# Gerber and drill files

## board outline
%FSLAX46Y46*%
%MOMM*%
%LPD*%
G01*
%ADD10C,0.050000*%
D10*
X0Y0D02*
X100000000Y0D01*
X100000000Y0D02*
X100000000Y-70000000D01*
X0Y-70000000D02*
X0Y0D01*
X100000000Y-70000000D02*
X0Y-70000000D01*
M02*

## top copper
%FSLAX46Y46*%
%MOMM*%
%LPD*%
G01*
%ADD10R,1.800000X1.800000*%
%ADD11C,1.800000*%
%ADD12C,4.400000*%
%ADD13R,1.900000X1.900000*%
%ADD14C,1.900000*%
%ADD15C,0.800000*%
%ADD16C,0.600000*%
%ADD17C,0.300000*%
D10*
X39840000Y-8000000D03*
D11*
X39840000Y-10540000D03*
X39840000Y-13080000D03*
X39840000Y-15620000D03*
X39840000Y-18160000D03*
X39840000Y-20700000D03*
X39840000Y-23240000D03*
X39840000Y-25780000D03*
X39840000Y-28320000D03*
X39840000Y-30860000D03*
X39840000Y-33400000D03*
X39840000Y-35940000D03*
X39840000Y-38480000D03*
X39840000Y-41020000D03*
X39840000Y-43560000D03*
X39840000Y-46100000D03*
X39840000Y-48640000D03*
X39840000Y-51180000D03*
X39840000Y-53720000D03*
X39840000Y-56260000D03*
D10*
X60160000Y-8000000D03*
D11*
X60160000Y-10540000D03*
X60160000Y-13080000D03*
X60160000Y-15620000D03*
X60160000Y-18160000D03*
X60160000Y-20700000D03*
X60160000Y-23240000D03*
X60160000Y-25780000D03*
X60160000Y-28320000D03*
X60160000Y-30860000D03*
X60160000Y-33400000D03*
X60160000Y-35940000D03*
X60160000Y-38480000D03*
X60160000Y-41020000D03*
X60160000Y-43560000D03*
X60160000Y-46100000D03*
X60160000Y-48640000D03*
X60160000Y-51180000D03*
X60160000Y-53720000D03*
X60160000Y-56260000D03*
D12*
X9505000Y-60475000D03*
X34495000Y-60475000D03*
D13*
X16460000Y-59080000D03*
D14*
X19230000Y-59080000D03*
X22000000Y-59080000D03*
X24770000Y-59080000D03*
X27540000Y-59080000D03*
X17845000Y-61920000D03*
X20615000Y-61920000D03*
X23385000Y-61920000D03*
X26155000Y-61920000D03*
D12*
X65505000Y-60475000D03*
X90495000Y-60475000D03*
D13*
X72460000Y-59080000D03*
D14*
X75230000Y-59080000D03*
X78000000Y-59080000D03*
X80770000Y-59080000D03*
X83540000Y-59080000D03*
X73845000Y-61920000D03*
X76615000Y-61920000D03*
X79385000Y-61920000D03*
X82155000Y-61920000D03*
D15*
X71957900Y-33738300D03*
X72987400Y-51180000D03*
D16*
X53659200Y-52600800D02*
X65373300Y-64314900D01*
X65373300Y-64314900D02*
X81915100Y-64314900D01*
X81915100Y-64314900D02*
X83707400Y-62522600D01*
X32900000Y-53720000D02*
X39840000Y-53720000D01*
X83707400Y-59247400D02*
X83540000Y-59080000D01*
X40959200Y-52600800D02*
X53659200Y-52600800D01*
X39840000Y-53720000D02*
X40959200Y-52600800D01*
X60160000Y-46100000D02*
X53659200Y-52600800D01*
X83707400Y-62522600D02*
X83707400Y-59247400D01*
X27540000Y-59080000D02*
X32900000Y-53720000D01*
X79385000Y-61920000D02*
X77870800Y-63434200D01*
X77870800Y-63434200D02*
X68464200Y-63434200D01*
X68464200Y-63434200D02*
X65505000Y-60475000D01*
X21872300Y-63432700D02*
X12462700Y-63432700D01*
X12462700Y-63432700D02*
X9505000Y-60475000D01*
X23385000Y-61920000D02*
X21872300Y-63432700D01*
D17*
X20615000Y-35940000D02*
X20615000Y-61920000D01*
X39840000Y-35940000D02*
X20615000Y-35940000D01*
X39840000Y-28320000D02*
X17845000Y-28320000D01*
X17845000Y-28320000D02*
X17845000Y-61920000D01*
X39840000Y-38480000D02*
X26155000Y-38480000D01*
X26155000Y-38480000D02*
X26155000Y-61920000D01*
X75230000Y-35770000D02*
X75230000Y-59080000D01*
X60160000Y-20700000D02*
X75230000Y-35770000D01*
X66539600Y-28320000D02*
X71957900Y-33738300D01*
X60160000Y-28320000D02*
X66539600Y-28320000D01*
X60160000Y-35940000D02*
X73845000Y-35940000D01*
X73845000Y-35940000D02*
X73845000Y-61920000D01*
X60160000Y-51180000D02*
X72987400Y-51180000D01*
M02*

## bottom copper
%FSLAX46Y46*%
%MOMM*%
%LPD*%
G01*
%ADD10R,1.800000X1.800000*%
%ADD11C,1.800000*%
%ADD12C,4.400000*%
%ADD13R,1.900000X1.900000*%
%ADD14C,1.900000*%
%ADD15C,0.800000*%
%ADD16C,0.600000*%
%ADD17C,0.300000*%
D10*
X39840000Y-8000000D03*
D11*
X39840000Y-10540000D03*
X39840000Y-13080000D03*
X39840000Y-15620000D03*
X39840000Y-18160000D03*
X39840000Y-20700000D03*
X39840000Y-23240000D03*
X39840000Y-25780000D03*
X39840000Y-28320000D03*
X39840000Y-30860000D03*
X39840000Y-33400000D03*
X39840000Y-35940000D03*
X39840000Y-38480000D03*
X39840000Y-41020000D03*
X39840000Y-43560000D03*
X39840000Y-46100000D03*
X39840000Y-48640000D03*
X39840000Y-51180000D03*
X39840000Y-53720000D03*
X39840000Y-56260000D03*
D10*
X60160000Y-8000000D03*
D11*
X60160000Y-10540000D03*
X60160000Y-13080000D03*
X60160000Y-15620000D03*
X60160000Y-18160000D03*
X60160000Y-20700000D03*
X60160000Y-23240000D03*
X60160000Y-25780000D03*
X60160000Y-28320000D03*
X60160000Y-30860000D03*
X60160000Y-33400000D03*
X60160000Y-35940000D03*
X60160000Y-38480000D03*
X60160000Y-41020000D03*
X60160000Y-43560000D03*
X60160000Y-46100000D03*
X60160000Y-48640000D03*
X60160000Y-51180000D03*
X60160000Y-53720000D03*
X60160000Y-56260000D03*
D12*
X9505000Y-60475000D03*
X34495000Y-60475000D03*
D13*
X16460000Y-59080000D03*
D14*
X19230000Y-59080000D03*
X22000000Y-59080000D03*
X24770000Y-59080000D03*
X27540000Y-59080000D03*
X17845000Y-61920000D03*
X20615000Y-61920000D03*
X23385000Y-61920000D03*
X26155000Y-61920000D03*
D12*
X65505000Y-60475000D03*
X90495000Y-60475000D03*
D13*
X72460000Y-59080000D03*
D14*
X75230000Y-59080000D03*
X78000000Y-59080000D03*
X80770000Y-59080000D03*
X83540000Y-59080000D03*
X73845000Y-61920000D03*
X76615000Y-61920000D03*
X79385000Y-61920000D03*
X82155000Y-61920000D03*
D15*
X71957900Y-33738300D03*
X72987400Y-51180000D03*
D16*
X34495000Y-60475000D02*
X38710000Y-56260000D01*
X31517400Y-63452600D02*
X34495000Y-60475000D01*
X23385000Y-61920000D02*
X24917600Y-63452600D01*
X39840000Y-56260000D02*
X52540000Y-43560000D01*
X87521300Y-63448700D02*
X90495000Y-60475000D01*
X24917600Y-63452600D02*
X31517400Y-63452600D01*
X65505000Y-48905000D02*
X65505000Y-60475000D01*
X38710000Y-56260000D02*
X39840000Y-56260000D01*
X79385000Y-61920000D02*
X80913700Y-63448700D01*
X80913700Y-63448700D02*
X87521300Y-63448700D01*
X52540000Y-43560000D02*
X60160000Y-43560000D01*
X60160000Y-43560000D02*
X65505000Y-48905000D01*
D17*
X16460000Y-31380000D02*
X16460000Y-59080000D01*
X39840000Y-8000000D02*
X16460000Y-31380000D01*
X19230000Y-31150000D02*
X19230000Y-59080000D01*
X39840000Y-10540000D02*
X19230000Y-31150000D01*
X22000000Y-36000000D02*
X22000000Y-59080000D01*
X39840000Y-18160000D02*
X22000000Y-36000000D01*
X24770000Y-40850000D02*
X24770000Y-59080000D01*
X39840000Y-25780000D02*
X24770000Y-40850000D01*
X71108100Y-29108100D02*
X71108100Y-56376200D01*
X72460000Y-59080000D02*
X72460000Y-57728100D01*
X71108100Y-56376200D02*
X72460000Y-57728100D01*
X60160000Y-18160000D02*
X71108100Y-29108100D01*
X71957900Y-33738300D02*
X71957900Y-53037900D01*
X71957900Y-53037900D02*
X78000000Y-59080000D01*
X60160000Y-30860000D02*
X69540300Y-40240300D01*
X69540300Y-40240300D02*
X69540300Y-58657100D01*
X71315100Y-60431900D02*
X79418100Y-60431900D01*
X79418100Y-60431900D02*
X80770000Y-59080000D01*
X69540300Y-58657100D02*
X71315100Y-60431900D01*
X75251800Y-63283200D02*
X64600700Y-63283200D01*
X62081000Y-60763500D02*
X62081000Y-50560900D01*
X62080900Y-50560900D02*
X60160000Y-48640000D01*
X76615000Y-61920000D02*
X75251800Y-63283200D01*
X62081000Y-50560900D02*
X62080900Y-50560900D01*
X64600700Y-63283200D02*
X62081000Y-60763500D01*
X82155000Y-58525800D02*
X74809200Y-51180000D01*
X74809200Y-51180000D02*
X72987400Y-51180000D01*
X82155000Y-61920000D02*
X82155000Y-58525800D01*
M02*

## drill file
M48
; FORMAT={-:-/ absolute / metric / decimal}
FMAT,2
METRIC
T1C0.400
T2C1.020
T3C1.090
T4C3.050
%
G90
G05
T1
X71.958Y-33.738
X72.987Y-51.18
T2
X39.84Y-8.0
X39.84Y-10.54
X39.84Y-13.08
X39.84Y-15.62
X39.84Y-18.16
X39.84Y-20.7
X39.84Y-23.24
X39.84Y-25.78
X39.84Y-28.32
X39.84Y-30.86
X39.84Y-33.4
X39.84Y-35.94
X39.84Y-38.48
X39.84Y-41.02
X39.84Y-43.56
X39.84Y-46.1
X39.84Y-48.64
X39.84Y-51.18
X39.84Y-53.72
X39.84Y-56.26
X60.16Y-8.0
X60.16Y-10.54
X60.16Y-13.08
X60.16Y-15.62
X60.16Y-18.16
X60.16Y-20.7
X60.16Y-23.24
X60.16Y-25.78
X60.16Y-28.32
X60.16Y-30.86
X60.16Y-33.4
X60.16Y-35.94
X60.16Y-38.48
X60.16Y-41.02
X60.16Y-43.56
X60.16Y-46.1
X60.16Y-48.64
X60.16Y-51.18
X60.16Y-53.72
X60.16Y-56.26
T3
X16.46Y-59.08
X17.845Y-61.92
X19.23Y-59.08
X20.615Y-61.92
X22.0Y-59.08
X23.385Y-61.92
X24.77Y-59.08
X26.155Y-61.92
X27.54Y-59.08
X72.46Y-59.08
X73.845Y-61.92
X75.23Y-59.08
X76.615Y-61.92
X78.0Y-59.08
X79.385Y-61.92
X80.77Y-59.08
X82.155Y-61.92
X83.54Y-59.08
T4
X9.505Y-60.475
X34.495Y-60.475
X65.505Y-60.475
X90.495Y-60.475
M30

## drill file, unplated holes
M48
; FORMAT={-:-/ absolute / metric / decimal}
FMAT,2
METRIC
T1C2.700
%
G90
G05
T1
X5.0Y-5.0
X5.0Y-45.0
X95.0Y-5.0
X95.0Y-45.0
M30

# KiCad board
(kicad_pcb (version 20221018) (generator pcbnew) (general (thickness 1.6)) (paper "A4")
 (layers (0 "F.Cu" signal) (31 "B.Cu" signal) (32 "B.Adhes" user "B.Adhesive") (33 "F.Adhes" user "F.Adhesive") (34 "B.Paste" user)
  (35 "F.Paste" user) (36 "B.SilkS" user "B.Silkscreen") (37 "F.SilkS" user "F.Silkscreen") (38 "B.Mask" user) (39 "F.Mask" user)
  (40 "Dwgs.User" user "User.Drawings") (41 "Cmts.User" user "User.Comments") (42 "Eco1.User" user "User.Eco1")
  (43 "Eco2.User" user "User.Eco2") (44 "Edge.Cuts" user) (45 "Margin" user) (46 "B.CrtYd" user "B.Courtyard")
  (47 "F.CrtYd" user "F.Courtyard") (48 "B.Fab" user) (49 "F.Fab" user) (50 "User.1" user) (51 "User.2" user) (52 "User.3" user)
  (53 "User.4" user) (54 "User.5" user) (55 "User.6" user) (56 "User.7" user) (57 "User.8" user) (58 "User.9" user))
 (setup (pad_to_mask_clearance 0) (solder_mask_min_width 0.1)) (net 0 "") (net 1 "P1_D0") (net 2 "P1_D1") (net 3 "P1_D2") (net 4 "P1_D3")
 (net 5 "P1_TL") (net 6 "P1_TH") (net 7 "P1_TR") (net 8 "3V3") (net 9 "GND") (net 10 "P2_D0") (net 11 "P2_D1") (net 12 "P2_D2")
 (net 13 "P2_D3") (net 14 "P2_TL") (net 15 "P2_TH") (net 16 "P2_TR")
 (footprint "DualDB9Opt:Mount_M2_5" (layer "F.Cu") (at 95 45)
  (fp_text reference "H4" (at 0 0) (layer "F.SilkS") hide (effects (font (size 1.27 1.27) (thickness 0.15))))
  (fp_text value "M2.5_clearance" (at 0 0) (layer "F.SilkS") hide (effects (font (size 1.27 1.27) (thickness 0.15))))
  (pad "" np_thru_hole circle (at 0 0) (size 2.7 2.7) (drill 2.7) (layers "F&B.Cu" "*.Mask")))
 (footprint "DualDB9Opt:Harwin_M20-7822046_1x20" (layer "F.Cu") (at 39.84 8)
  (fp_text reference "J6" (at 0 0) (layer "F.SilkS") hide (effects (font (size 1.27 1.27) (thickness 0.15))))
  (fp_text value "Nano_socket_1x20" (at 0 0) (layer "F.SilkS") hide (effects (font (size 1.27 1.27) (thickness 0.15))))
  (pad "1" thru_hole rect (at 0 0) (size 1.8 1.8) (drill 1.02) (layers "F&B.Cu" "*.Mask") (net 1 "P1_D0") (thermal_bridge_angle 45))
  (pad "2" thru_hole circle (at 0 2.54) (size 1.8 1.8) (drill 1.02) (layers "F&B.Cu" "*.Mask") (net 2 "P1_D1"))
  (pad "3" thru_hole circle (at 0 5.08) (size 1.8 1.8) (drill 1.02) (layers "F&B.Cu" "*.Mask"))
  (pad "4" thru_hole circle (at 0 7.62) (size 1.8 1.8) (drill 1.02) (layers "F&B.Cu" "*.Mask"))
  (pad "5" thru_hole circle (at 0 10.16) (size 1.8 1.8) (drill 1.02) (layers "F&B.Cu" "*.Mask") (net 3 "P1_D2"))
  (pad "6" thru_hole circle (at 0 12.7) (size 1.8 1.8) (drill 1.02) (layers "F&B.Cu" "*.Mask"))
  (pad "7" thru_hole circle (at 0 15.24) (size 1.8 1.8) (drill 1.02) (layers "F&B.Cu" "*.Mask"))
  (pad "8" thru_hole circle (at 0 17.78) (size 1.8 1.8) (drill 1.02) (layers "F&B.Cu" "*.Mask") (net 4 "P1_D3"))
  (pad "9" thru_hole circle (at 0 20.32) (size 1.8 1.8) (drill 1.02) (layers "F&B.Cu" "*.Mask") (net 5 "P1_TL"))
  (pad "10" thru_hole circle (at 0 22.86) (size 1.8 1.8) (drill 1.02) (layers "F&B.Cu" "*.Mask"))
  (pad "11" thru_hole circle (at 0 25.4) (size 1.8 1.8) (drill 1.02) (layers "F&B.Cu" "*.Mask"))
  (pad "12" thru_hole circle (at 0 27.94) (size 1.8 1.8) (drill 1.02) (layers "F&B.Cu" "*.Mask") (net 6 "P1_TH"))
  (pad "13" thru_hole circle (at 0 30.48) (size 1.8 1.8) (drill 1.02) (layers "F&B.Cu" "*.Mask") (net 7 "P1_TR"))
  (pad "14" thru_hole circle (at 0 33.02) (size 1.8 1.8) (drill 1.02) (layers "F&B.Cu" "*.Mask"))
  (pad "15" thru_hole circle (at 0 35.56) (size 1.8 1.8) (drill 1.02) (layers "F&B.Cu" "*.Mask"))
  (pad "16" thru_hole circle (at 0 38.1) (size 1.8 1.8) (drill 1.02) (layers "F&B.Cu" "*.Mask"))
  (pad "17" thru_hole circle (at 0 40.64) (size 1.8 1.8) (drill 1.02) (layers "F&B.Cu" "*.Mask"))
  (pad "18" thru_hole circle (at 0 43.18) (size 1.8 1.8) (drill 1.02) (layers "F&B.Cu" "*.Mask"))
  (pad "19" thru_hole circle (at 0 45.72) (size 1.8 1.8) (drill 1.02) (layers "F&B.Cu" "*.Mask") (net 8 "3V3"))
  (pad "20" thru_hole circle (at 0 48.26) (size 1.8 1.8) (drill 1.02) (layers "F&B.Cu" "*.Mask") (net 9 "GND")))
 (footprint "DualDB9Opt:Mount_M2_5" (layer "F.Cu") (at 5 5)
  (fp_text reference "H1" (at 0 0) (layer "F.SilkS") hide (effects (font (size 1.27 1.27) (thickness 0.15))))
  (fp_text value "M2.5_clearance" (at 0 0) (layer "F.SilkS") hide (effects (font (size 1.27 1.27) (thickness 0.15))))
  (pad "" np_thru_hole circle (at 0 0) (size 2.7 2.7) (drill 2.7) (layers "F&B.Cu" "*.Mask")))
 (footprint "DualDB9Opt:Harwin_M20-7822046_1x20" (layer "F.Cu") (at 60.16 8)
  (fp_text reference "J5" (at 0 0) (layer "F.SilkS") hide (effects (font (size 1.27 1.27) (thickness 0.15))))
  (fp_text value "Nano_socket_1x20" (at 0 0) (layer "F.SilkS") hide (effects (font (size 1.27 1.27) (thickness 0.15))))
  (pad "1" thru_hole rect (at 0 0) (size 1.8 1.8) (drill 1.02) (layers "F&B.Cu" "*.Mask") (thermal_bridge_angle 45))
  (pad "2" thru_hole circle (at 0 2.54) (size 1.8 1.8) (drill 1.02) (layers "F&B.Cu" "*.Mask"))
  (pad "3" thru_hole circle (at 0 5.08) (size 1.8 1.8) (drill 1.02) (layers "F&B.Cu" "*.Mask"))
  (pad "4" thru_hole circle (at 0 7.62) (size 1.8 1.8) (drill 1.02) (layers "F&B.Cu" "*.Mask"))
  (pad "5" thru_hole circle (at 0 10.16) (size 1.8 1.8) (drill 1.02) (layers "F&B.Cu" "*.Mask") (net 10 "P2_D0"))
  (pad "6" thru_hole circle (at 0 12.7) (size 1.8 1.8) (drill 1.02) (layers "F&B.Cu" "*.Mask") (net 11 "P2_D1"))
  (pad "7" thru_hole circle (at 0 15.24) (size 1.8 1.8) (drill 1.02) (layers "F&B.Cu" "*.Mask"))
  (pad "8" thru_hole circle (at 0 17.78) (size 1.8 1.8) (drill 1.02) (layers "F&B.Cu" "*.Mask"))
  (pad "9" thru_hole circle (at 0 20.32) (size 1.8 1.8) (drill 1.02) (layers "F&B.Cu" "*.Mask") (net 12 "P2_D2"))
  (pad "10" thru_hole circle (at 0 22.86) (size 1.8 1.8) (drill 1.02) (layers "F&B.Cu" "*.Mask") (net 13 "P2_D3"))
  (pad "11" thru_hole circle (at 0 25.4) (size 1.8 1.8) (drill 1.02) (layers "F&B.Cu" "*.Mask"))
  (pad "12" thru_hole circle (at 0 27.94) (size 1.8 1.8) (drill 1.02) (layers "F&B.Cu" "*.Mask") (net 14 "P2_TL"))
  (pad "13" thru_hole circle (at 0 30.48) (size 1.8 1.8) (drill 1.02) (layers "F&B.Cu" "*.Mask"))
  (pad "14" thru_hole circle (at 0 33.02) (size 1.8 1.8) (drill 1.02) (layers "F&B.Cu" "*.Mask"))
  (pad "15" thru_hole circle (at 0 35.56) (size 1.8 1.8) (drill 1.02) (layers "F&B.Cu" "*.Mask") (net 9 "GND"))
  (pad "16" thru_hole circle (at 0 38.1) (size 1.8 1.8) (drill 1.02) (layers "F&B.Cu" "*.Mask") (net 8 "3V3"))
  (pad "17" thru_hole circle (at 0 40.64) (size 1.8 1.8) (drill 1.02) (layers "F&B.Cu" "*.Mask") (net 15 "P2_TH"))
  (pad "18" thru_hole circle (at 0 43.18) (size 1.8 1.8) (drill 1.02) (layers "F&B.Cu" "*.Mask") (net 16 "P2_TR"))
  (pad "19" thru_hole circle (at 0 45.72) (size 1.8 1.8) (drill 1.02) (layers "F&B.Cu" "*.Mask"))
  (pad "20" thru_hole circle (at 0 48.26) (size 1.8 1.8) (drill 1.02) (layers "F&B.Cu" "*.Mask")))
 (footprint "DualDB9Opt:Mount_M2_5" (layer "F.Cu") (at 5 45)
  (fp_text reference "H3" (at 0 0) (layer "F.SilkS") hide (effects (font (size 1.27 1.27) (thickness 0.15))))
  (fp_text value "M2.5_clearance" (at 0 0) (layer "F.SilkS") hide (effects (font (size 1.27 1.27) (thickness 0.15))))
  (pad "" np_thru_hole circle (at 0 0) (size 2.7 2.7) (drill 2.7) (layers "F&B.Cu" "*.Mask")))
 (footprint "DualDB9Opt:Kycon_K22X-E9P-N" (layer "F.Cu") (at 16.46 59.08)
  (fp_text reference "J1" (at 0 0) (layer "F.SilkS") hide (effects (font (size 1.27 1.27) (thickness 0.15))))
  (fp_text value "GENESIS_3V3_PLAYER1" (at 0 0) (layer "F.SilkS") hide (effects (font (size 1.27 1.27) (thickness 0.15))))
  (pad "0" thru_hole circle (at -6.955 1.395) (size 4.4 4.4) (drill 3.05) (layers "F&B.Cu" "*.Mask") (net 9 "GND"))
  (pad "0" thru_hole circle (at 18.035 1.395) (size 4.4 4.4) (drill 3.05) (layers "F&B.Cu" "*.Mask") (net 9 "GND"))
  (pad "1" thru_hole rect (at 0 0) (size 1.9 1.9) (drill 1.09) (layers "F&B.Cu" "*.Mask") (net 1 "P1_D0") (thermal_bridge_angle 45))
  (pad "2" thru_hole circle (at 2.77 0) (size 1.9 1.9) (drill 1.09) (layers "F&B.Cu" "*.Mask") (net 2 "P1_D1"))
  (pad "3" thru_hole circle (at 5.54 0) (size 1.9 1.9) (drill 1.09) (layers "F&B.Cu" "*.Mask") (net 3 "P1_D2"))
  (pad "4" thru_hole circle (at 8.31 0) (size 1.9 1.9) (drill 1.09) (layers "F&B.Cu" "*.Mask") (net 4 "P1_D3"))
  (pad "5" thru_hole circle (at 11.08 0) (size 1.9 1.9) (drill 1.09) (layers "F&B.Cu" "*.Mask") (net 8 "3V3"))
  (pad "6" thru_hole circle (at 1.385 2.84) (size 1.9 1.9) (drill 1.09) (layers "F&B.Cu" "*.Mask") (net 5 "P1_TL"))
  (pad "7" thru_hole circle (at 4.155 2.84) (size 1.9 1.9) (drill 1.09) (layers "F&B.Cu" "*.Mask") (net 6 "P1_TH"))
  (pad "8" thru_hole circle (at 6.925 2.84) (size 1.9 1.9) (drill 1.09) (layers "F&B.Cu" "*.Mask") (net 9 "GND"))
  (pad "9" thru_hole circle (at 9.695 2.84) (size 1.9 1.9) (drill 1.09) (layers "F&B.Cu" "*.Mask") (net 7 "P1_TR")))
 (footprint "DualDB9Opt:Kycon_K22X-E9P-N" (layer "F.Cu") (at 72.46 59.08)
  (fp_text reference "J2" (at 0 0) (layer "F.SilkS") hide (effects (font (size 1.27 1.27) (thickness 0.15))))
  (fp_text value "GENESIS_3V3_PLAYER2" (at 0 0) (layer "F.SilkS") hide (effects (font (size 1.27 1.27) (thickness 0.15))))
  (pad "0" thru_hole circle (at -6.955 1.395) (size 4.4 4.4) (drill 3.05) (layers "F&B.Cu" "*.Mask") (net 9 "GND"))
  (pad "0" thru_hole circle (at 18.035 1.395) (size 4.4 4.4) (drill 3.05) (layers "F&B.Cu" "*.Mask") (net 9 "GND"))
  (pad "1" thru_hole rect (at 0 0) (size 1.9 1.9) (drill 1.09) (layers "F&B.Cu" "*.Mask") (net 10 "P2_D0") (thermal_bridge_angle 45))
  (pad "2" thru_hole circle (at 2.77 0) (size 1.9 1.9) (drill 1.09) (layers "F&B.Cu" "*.Mask") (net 11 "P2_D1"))
  (pad "3" thru_hole circle (at 5.54 0) (size 1.9 1.9) (drill 1.09) (layers "F&B.Cu" "*.Mask") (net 12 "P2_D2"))
  (pad "4" thru_hole circle (at 8.31 0) (size 1.9 1.9) (drill 1.09) (layers "F&B.Cu" "*.Mask") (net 13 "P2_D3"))
  (pad "5" thru_hole circle (at 11.08 0) (size 1.9 1.9) (drill 1.09) (layers "F&B.Cu" "*.Mask") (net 8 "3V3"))
  (pad "6" thru_hole circle (at 1.385 2.84) (size 1.9 1.9) (drill 1.09) (layers "F&B.Cu" "*.Mask") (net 14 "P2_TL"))
  (pad "7" thru_hole circle (at 4.155 2.84) (size 1.9 1.9) (drill 1.09) (layers "F&B.Cu" "*.Mask") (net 15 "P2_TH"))
  (pad "8" thru_hole circle (at 6.925 2.84) (size 1.9 1.9) (drill 1.09) (layers "F&B.Cu" "*.Mask") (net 9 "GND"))
  (pad "9" thru_hole circle (at 9.695 2.84) (size 1.9 1.9) (drill 1.09) (layers "F&B.Cu" "*.Mask") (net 16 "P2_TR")))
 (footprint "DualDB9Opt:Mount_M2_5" (layer "F.Cu") (at 95 5)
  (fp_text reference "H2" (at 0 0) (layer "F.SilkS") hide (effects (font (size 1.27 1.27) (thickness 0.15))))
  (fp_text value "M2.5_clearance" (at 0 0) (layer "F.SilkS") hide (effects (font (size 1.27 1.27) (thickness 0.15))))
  (pad "" np_thru_hole circle (at 0 0) (size 2.7 2.7) (drill 2.7) (layers "F&B.Cu" "*.Mask")))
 (gr_line (start 0 0) (end 100 0) (stroke (width 0.05) (type default)) (layer "Edge.Cuts"))
 (gr_line (start 100 0) (end 100 70) (stroke (width 0.05) (type default)) (layer "Edge.Cuts"))
 (gr_line (start 0 70) (end 0 0) (stroke (width 0.05) (type default)) (layer "Edge.Cuts"))
 (gr_line (start 100 70) (end 0 70) (stroke (width 0.05) (type default)) (layer "Edge.Cuts"))
 (segment (start 53.6592 52.6008) (end 65.3733 64.3149) (width 0.6) (layer "F.Cu") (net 8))
 (segment (start 65.3733 64.3149) (end 81.9151 64.3149) (width 0.6) (layer "F.Cu") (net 8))
 (segment (start 81.9151 64.3149) (end 83.7074 62.5226) (width 0.6) (layer "F.Cu") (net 8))
 (segment (start 32.9 53.72) (end 39.84 53.72) (width 0.6) (layer "F.Cu") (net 8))
 (segment (start 83.7074 59.2474) (end 83.54 59.08) (width 0.6) (layer "F.Cu") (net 8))
 (segment (start 40.9592 52.6008) (end 53.6592 52.6008) (width 0.6) (layer "F.Cu") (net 8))
 (segment (start 39.84 53.72) (end 40.9592 52.6008) (width 0.6) (layer "F.Cu") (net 8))
 (segment (start 60.16 46.1) (end 53.6592 52.6008) (width 0.6) (layer "F.Cu") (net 8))
 (segment (start 83.7074 62.5226) (end 83.7074 59.2474) (width 0.6) (layer "F.Cu") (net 8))
 (segment (start 27.54 59.08) (end 32.9 53.72) (width 0.6) (layer "F.Cu") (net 8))
 (segment (start 79.385 61.92) (end 77.8708 63.4342) (width 0.6) (layer "F.Cu") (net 9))
 (segment (start 77.8708 63.4342) (end 68.4642 63.4342) (width 0.6) (layer "F.Cu") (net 9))
 (segment (start 68.4642 63.4342) (end 65.505 60.475) (width 0.6) (layer "F.Cu") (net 9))
 (segment (start 21.8723 63.4327) (end 12.4627 63.4327) (width 0.6) (layer "F.Cu") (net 9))
 (segment (start 12.4627 63.4327) (end 9.505 60.475) (width 0.6) (layer "F.Cu") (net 9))
 (segment (start 23.385 61.92) (end 21.8723 63.4327) (width 0.6) (layer "F.Cu") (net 9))
 (segment (start 34.495 60.475) (end 38.71 56.26) (width 0.6) (layer "B.Cu") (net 9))
 (segment (start 31.5174 63.4526) (end 34.495 60.475) (width 0.6) (layer "B.Cu") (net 9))
 (segment (start 23.385 61.92) (end 24.9176 63.4526) (width 0.6) (layer "B.Cu") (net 9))
 (segment (start 39.84 56.26) (end 52.54 43.56) (width 0.6) (layer "B.Cu") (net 9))
 (segment (start 87.5213 63.4487) (end 90.495 60.475) (width 0.6) (layer "B.Cu") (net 9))
 (segment (start 24.9176 63.4526) (end 31.5174 63.4526) (width 0.6) (layer "B.Cu") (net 9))
 (segment (start 65.505 48.905) (end 65.505 60.475) (width 0.6) (layer "B.Cu") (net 9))
 (segment (start 38.71 56.26) (end 39.84 56.26) (width 0.6) (layer "B.Cu") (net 9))
 (segment (start 79.385 61.92) (end 80.9137 63.4487) (width 0.6) (layer "B.Cu") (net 9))
 (segment (start 80.9137 63.4487) (end 87.5213 63.4487) (width 0.6) (layer "B.Cu") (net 9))
 (segment (start 52.54 43.56) (end 60.16 43.56) (width 0.6) (layer "B.Cu") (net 9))
 (segment (start 60.16 43.56) (end 65.505 48.905) (width 0.6) (layer "B.Cu") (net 9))
 (segment (start 16.46 31.38) (end 16.46 59.08) (width 0.3) (layer "B.Cu") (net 1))
 (segment (start 39.84 8) (end 16.46 31.38) (width 0.3) (layer "B.Cu") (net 1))
 (segment (start 19.23 31.15) (end 19.23 59.08) (width 0.3) (layer "B.Cu") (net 2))
 (segment (start 39.84 10.54) (end 19.23 31.15) (width 0.3) (layer "B.Cu") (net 2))
 (segment (start 22 36) (end 22 59.08) (width 0.3) (layer "B.Cu") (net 3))
 (segment (start 39.84 18.16) (end 22 36) (width 0.3) (layer "B.Cu") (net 3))
 (segment (start 24.77 40.85) (end 24.77 59.08) (width 0.3) (layer "B.Cu") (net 4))
 (segment (start 39.84 25.78) (end 24.77 40.85) (width 0.3) (layer "B.Cu") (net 4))
 (segment (start 20.615 35.94) (end 20.615 61.92) (width 0.3) (layer "F.Cu") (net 6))
 (segment (start 39.84 35.94) (end 20.615 35.94) (width 0.3) (layer "F.Cu") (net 6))
 (segment (start 39.84 28.32) (end 17.845 28.32) (width 0.3) (layer "F.Cu") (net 5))
 (segment (start 17.845 28.32) (end 17.845 61.92) (width 0.3) (layer "F.Cu") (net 5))
 (segment (start 39.84 38.48) (end 26.155 38.48) (width 0.3) (layer "F.Cu") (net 7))
 (segment (start 26.155 38.48) (end 26.155 61.92) (width 0.3) (layer "F.Cu") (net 7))
 (segment (start 71.1081 29.1081) (end 71.1081 56.3762) (width 0.3) (layer "B.Cu") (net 10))
 (segment (start 72.46 59.08) (end 72.46 57.7281) (width 0.3) (layer "B.Cu") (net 10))
 (segment (start 71.1081 56.3762) (end 72.46 57.7281) (width 0.3) (layer "B.Cu") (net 10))
 (segment (start 60.16 18.16) (end 71.1081 29.1081) (width 0.3) (layer "B.Cu") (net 10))
 (segment (start 75.23 35.77) (end 75.23 59.08) (width 0.3) (layer "F.Cu") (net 11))
 (segment (start 60.16 20.7) (end 75.23 35.77) (width 0.3) (layer "F.Cu") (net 11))
 (segment (start 66.5396 28.32) (end 71.9579 33.7383) (width 0.3) (layer "F.Cu") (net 12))
 (segment (start 60.16 28.32) (end 66.5396 28.32) (width 0.3) (layer "F.Cu") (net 12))
 (via (at 71.9579 33.7383) (size 0.8) (drill 0.4) (layers "F.Cu" "B.Cu") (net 12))
 (segment (start 71.9579 33.7383) (end 71.9579 53.0379) (width 0.3) (layer "B.Cu") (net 12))
 (segment (start 71.9579 53.0379) (end 78 59.08) (width 0.3) (layer "B.Cu") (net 12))
 (segment (start 60.16 30.86) (end 69.5403 40.2403) (width 0.3) (layer "B.Cu") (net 13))
 (segment (start 69.5403 40.2403) (end 69.5403 58.6571) (width 0.3) (layer "B.Cu") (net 13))
 (segment (start 71.3151 60.4319) (end 79.4181 60.4319) (width 0.3) (layer "B.Cu") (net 13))
 (segment (start 79.4181 60.4319) (end 80.77 59.08) (width 0.3) (layer "B.Cu") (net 13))
 (segment (start 69.5403 58.6571) (end 71.3151 60.4319) (width 0.3) (layer "B.Cu") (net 13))
 (segment (start 75.2518 63.2832) (end 64.6007 63.2832) (width 0.3) (layer "B.Cu") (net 15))
 (segment (start 62.081 60.7635) (end 62.081 50.5609) (width 0.3) (layer "B.Cu") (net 15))
 (segment (start 62.0809 50.5609) (end 60.16 48.64) (width 0.3) (layer "B.Cu") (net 15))
 (segment (start 76.615 61.92) (end 75.2518 63.2832) (width 0.3) (layer "B.Cu") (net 15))
 (segment (start 62.081 50.5609) (end 62.0809 50.5609) (width 0.3) (layer "B.Cu") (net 15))
 (segment (start 64.6007 63.2832) (end 62.081 60.7635) (width 0.3) (layer "B.Cu") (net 15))
 (segment (start 60.16 35.94) (end 73.845 35.94) (width 0.3) (layer "F.Cu") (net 14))
 (segment (start 73.845 35.94) (end 73.845 61.92) (width 0.3) (layer "F.Cu") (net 14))
 (segment (start 60.16 51.18) (end 72.9874 51.18) (width 0.3) (layer "F.Cu") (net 16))
 (via (at 72.9874 51.18) (size 0.8) (drill 0.4) (layers "F.Cu" "B.Cu") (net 16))
 (segment (start 82.155 58.5258) (end 74.8092 51.18) (width 0.3) (layer "B.Cu") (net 16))
 (segment (start 74.8092 51.18) (end 72.9874 51.18) (width 0.3) (layer "B.Cu") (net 16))
 (segment (start 82.155 61.92) (end 82.155 58.5258) (width 0.3) (layer "B.Cu") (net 16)))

